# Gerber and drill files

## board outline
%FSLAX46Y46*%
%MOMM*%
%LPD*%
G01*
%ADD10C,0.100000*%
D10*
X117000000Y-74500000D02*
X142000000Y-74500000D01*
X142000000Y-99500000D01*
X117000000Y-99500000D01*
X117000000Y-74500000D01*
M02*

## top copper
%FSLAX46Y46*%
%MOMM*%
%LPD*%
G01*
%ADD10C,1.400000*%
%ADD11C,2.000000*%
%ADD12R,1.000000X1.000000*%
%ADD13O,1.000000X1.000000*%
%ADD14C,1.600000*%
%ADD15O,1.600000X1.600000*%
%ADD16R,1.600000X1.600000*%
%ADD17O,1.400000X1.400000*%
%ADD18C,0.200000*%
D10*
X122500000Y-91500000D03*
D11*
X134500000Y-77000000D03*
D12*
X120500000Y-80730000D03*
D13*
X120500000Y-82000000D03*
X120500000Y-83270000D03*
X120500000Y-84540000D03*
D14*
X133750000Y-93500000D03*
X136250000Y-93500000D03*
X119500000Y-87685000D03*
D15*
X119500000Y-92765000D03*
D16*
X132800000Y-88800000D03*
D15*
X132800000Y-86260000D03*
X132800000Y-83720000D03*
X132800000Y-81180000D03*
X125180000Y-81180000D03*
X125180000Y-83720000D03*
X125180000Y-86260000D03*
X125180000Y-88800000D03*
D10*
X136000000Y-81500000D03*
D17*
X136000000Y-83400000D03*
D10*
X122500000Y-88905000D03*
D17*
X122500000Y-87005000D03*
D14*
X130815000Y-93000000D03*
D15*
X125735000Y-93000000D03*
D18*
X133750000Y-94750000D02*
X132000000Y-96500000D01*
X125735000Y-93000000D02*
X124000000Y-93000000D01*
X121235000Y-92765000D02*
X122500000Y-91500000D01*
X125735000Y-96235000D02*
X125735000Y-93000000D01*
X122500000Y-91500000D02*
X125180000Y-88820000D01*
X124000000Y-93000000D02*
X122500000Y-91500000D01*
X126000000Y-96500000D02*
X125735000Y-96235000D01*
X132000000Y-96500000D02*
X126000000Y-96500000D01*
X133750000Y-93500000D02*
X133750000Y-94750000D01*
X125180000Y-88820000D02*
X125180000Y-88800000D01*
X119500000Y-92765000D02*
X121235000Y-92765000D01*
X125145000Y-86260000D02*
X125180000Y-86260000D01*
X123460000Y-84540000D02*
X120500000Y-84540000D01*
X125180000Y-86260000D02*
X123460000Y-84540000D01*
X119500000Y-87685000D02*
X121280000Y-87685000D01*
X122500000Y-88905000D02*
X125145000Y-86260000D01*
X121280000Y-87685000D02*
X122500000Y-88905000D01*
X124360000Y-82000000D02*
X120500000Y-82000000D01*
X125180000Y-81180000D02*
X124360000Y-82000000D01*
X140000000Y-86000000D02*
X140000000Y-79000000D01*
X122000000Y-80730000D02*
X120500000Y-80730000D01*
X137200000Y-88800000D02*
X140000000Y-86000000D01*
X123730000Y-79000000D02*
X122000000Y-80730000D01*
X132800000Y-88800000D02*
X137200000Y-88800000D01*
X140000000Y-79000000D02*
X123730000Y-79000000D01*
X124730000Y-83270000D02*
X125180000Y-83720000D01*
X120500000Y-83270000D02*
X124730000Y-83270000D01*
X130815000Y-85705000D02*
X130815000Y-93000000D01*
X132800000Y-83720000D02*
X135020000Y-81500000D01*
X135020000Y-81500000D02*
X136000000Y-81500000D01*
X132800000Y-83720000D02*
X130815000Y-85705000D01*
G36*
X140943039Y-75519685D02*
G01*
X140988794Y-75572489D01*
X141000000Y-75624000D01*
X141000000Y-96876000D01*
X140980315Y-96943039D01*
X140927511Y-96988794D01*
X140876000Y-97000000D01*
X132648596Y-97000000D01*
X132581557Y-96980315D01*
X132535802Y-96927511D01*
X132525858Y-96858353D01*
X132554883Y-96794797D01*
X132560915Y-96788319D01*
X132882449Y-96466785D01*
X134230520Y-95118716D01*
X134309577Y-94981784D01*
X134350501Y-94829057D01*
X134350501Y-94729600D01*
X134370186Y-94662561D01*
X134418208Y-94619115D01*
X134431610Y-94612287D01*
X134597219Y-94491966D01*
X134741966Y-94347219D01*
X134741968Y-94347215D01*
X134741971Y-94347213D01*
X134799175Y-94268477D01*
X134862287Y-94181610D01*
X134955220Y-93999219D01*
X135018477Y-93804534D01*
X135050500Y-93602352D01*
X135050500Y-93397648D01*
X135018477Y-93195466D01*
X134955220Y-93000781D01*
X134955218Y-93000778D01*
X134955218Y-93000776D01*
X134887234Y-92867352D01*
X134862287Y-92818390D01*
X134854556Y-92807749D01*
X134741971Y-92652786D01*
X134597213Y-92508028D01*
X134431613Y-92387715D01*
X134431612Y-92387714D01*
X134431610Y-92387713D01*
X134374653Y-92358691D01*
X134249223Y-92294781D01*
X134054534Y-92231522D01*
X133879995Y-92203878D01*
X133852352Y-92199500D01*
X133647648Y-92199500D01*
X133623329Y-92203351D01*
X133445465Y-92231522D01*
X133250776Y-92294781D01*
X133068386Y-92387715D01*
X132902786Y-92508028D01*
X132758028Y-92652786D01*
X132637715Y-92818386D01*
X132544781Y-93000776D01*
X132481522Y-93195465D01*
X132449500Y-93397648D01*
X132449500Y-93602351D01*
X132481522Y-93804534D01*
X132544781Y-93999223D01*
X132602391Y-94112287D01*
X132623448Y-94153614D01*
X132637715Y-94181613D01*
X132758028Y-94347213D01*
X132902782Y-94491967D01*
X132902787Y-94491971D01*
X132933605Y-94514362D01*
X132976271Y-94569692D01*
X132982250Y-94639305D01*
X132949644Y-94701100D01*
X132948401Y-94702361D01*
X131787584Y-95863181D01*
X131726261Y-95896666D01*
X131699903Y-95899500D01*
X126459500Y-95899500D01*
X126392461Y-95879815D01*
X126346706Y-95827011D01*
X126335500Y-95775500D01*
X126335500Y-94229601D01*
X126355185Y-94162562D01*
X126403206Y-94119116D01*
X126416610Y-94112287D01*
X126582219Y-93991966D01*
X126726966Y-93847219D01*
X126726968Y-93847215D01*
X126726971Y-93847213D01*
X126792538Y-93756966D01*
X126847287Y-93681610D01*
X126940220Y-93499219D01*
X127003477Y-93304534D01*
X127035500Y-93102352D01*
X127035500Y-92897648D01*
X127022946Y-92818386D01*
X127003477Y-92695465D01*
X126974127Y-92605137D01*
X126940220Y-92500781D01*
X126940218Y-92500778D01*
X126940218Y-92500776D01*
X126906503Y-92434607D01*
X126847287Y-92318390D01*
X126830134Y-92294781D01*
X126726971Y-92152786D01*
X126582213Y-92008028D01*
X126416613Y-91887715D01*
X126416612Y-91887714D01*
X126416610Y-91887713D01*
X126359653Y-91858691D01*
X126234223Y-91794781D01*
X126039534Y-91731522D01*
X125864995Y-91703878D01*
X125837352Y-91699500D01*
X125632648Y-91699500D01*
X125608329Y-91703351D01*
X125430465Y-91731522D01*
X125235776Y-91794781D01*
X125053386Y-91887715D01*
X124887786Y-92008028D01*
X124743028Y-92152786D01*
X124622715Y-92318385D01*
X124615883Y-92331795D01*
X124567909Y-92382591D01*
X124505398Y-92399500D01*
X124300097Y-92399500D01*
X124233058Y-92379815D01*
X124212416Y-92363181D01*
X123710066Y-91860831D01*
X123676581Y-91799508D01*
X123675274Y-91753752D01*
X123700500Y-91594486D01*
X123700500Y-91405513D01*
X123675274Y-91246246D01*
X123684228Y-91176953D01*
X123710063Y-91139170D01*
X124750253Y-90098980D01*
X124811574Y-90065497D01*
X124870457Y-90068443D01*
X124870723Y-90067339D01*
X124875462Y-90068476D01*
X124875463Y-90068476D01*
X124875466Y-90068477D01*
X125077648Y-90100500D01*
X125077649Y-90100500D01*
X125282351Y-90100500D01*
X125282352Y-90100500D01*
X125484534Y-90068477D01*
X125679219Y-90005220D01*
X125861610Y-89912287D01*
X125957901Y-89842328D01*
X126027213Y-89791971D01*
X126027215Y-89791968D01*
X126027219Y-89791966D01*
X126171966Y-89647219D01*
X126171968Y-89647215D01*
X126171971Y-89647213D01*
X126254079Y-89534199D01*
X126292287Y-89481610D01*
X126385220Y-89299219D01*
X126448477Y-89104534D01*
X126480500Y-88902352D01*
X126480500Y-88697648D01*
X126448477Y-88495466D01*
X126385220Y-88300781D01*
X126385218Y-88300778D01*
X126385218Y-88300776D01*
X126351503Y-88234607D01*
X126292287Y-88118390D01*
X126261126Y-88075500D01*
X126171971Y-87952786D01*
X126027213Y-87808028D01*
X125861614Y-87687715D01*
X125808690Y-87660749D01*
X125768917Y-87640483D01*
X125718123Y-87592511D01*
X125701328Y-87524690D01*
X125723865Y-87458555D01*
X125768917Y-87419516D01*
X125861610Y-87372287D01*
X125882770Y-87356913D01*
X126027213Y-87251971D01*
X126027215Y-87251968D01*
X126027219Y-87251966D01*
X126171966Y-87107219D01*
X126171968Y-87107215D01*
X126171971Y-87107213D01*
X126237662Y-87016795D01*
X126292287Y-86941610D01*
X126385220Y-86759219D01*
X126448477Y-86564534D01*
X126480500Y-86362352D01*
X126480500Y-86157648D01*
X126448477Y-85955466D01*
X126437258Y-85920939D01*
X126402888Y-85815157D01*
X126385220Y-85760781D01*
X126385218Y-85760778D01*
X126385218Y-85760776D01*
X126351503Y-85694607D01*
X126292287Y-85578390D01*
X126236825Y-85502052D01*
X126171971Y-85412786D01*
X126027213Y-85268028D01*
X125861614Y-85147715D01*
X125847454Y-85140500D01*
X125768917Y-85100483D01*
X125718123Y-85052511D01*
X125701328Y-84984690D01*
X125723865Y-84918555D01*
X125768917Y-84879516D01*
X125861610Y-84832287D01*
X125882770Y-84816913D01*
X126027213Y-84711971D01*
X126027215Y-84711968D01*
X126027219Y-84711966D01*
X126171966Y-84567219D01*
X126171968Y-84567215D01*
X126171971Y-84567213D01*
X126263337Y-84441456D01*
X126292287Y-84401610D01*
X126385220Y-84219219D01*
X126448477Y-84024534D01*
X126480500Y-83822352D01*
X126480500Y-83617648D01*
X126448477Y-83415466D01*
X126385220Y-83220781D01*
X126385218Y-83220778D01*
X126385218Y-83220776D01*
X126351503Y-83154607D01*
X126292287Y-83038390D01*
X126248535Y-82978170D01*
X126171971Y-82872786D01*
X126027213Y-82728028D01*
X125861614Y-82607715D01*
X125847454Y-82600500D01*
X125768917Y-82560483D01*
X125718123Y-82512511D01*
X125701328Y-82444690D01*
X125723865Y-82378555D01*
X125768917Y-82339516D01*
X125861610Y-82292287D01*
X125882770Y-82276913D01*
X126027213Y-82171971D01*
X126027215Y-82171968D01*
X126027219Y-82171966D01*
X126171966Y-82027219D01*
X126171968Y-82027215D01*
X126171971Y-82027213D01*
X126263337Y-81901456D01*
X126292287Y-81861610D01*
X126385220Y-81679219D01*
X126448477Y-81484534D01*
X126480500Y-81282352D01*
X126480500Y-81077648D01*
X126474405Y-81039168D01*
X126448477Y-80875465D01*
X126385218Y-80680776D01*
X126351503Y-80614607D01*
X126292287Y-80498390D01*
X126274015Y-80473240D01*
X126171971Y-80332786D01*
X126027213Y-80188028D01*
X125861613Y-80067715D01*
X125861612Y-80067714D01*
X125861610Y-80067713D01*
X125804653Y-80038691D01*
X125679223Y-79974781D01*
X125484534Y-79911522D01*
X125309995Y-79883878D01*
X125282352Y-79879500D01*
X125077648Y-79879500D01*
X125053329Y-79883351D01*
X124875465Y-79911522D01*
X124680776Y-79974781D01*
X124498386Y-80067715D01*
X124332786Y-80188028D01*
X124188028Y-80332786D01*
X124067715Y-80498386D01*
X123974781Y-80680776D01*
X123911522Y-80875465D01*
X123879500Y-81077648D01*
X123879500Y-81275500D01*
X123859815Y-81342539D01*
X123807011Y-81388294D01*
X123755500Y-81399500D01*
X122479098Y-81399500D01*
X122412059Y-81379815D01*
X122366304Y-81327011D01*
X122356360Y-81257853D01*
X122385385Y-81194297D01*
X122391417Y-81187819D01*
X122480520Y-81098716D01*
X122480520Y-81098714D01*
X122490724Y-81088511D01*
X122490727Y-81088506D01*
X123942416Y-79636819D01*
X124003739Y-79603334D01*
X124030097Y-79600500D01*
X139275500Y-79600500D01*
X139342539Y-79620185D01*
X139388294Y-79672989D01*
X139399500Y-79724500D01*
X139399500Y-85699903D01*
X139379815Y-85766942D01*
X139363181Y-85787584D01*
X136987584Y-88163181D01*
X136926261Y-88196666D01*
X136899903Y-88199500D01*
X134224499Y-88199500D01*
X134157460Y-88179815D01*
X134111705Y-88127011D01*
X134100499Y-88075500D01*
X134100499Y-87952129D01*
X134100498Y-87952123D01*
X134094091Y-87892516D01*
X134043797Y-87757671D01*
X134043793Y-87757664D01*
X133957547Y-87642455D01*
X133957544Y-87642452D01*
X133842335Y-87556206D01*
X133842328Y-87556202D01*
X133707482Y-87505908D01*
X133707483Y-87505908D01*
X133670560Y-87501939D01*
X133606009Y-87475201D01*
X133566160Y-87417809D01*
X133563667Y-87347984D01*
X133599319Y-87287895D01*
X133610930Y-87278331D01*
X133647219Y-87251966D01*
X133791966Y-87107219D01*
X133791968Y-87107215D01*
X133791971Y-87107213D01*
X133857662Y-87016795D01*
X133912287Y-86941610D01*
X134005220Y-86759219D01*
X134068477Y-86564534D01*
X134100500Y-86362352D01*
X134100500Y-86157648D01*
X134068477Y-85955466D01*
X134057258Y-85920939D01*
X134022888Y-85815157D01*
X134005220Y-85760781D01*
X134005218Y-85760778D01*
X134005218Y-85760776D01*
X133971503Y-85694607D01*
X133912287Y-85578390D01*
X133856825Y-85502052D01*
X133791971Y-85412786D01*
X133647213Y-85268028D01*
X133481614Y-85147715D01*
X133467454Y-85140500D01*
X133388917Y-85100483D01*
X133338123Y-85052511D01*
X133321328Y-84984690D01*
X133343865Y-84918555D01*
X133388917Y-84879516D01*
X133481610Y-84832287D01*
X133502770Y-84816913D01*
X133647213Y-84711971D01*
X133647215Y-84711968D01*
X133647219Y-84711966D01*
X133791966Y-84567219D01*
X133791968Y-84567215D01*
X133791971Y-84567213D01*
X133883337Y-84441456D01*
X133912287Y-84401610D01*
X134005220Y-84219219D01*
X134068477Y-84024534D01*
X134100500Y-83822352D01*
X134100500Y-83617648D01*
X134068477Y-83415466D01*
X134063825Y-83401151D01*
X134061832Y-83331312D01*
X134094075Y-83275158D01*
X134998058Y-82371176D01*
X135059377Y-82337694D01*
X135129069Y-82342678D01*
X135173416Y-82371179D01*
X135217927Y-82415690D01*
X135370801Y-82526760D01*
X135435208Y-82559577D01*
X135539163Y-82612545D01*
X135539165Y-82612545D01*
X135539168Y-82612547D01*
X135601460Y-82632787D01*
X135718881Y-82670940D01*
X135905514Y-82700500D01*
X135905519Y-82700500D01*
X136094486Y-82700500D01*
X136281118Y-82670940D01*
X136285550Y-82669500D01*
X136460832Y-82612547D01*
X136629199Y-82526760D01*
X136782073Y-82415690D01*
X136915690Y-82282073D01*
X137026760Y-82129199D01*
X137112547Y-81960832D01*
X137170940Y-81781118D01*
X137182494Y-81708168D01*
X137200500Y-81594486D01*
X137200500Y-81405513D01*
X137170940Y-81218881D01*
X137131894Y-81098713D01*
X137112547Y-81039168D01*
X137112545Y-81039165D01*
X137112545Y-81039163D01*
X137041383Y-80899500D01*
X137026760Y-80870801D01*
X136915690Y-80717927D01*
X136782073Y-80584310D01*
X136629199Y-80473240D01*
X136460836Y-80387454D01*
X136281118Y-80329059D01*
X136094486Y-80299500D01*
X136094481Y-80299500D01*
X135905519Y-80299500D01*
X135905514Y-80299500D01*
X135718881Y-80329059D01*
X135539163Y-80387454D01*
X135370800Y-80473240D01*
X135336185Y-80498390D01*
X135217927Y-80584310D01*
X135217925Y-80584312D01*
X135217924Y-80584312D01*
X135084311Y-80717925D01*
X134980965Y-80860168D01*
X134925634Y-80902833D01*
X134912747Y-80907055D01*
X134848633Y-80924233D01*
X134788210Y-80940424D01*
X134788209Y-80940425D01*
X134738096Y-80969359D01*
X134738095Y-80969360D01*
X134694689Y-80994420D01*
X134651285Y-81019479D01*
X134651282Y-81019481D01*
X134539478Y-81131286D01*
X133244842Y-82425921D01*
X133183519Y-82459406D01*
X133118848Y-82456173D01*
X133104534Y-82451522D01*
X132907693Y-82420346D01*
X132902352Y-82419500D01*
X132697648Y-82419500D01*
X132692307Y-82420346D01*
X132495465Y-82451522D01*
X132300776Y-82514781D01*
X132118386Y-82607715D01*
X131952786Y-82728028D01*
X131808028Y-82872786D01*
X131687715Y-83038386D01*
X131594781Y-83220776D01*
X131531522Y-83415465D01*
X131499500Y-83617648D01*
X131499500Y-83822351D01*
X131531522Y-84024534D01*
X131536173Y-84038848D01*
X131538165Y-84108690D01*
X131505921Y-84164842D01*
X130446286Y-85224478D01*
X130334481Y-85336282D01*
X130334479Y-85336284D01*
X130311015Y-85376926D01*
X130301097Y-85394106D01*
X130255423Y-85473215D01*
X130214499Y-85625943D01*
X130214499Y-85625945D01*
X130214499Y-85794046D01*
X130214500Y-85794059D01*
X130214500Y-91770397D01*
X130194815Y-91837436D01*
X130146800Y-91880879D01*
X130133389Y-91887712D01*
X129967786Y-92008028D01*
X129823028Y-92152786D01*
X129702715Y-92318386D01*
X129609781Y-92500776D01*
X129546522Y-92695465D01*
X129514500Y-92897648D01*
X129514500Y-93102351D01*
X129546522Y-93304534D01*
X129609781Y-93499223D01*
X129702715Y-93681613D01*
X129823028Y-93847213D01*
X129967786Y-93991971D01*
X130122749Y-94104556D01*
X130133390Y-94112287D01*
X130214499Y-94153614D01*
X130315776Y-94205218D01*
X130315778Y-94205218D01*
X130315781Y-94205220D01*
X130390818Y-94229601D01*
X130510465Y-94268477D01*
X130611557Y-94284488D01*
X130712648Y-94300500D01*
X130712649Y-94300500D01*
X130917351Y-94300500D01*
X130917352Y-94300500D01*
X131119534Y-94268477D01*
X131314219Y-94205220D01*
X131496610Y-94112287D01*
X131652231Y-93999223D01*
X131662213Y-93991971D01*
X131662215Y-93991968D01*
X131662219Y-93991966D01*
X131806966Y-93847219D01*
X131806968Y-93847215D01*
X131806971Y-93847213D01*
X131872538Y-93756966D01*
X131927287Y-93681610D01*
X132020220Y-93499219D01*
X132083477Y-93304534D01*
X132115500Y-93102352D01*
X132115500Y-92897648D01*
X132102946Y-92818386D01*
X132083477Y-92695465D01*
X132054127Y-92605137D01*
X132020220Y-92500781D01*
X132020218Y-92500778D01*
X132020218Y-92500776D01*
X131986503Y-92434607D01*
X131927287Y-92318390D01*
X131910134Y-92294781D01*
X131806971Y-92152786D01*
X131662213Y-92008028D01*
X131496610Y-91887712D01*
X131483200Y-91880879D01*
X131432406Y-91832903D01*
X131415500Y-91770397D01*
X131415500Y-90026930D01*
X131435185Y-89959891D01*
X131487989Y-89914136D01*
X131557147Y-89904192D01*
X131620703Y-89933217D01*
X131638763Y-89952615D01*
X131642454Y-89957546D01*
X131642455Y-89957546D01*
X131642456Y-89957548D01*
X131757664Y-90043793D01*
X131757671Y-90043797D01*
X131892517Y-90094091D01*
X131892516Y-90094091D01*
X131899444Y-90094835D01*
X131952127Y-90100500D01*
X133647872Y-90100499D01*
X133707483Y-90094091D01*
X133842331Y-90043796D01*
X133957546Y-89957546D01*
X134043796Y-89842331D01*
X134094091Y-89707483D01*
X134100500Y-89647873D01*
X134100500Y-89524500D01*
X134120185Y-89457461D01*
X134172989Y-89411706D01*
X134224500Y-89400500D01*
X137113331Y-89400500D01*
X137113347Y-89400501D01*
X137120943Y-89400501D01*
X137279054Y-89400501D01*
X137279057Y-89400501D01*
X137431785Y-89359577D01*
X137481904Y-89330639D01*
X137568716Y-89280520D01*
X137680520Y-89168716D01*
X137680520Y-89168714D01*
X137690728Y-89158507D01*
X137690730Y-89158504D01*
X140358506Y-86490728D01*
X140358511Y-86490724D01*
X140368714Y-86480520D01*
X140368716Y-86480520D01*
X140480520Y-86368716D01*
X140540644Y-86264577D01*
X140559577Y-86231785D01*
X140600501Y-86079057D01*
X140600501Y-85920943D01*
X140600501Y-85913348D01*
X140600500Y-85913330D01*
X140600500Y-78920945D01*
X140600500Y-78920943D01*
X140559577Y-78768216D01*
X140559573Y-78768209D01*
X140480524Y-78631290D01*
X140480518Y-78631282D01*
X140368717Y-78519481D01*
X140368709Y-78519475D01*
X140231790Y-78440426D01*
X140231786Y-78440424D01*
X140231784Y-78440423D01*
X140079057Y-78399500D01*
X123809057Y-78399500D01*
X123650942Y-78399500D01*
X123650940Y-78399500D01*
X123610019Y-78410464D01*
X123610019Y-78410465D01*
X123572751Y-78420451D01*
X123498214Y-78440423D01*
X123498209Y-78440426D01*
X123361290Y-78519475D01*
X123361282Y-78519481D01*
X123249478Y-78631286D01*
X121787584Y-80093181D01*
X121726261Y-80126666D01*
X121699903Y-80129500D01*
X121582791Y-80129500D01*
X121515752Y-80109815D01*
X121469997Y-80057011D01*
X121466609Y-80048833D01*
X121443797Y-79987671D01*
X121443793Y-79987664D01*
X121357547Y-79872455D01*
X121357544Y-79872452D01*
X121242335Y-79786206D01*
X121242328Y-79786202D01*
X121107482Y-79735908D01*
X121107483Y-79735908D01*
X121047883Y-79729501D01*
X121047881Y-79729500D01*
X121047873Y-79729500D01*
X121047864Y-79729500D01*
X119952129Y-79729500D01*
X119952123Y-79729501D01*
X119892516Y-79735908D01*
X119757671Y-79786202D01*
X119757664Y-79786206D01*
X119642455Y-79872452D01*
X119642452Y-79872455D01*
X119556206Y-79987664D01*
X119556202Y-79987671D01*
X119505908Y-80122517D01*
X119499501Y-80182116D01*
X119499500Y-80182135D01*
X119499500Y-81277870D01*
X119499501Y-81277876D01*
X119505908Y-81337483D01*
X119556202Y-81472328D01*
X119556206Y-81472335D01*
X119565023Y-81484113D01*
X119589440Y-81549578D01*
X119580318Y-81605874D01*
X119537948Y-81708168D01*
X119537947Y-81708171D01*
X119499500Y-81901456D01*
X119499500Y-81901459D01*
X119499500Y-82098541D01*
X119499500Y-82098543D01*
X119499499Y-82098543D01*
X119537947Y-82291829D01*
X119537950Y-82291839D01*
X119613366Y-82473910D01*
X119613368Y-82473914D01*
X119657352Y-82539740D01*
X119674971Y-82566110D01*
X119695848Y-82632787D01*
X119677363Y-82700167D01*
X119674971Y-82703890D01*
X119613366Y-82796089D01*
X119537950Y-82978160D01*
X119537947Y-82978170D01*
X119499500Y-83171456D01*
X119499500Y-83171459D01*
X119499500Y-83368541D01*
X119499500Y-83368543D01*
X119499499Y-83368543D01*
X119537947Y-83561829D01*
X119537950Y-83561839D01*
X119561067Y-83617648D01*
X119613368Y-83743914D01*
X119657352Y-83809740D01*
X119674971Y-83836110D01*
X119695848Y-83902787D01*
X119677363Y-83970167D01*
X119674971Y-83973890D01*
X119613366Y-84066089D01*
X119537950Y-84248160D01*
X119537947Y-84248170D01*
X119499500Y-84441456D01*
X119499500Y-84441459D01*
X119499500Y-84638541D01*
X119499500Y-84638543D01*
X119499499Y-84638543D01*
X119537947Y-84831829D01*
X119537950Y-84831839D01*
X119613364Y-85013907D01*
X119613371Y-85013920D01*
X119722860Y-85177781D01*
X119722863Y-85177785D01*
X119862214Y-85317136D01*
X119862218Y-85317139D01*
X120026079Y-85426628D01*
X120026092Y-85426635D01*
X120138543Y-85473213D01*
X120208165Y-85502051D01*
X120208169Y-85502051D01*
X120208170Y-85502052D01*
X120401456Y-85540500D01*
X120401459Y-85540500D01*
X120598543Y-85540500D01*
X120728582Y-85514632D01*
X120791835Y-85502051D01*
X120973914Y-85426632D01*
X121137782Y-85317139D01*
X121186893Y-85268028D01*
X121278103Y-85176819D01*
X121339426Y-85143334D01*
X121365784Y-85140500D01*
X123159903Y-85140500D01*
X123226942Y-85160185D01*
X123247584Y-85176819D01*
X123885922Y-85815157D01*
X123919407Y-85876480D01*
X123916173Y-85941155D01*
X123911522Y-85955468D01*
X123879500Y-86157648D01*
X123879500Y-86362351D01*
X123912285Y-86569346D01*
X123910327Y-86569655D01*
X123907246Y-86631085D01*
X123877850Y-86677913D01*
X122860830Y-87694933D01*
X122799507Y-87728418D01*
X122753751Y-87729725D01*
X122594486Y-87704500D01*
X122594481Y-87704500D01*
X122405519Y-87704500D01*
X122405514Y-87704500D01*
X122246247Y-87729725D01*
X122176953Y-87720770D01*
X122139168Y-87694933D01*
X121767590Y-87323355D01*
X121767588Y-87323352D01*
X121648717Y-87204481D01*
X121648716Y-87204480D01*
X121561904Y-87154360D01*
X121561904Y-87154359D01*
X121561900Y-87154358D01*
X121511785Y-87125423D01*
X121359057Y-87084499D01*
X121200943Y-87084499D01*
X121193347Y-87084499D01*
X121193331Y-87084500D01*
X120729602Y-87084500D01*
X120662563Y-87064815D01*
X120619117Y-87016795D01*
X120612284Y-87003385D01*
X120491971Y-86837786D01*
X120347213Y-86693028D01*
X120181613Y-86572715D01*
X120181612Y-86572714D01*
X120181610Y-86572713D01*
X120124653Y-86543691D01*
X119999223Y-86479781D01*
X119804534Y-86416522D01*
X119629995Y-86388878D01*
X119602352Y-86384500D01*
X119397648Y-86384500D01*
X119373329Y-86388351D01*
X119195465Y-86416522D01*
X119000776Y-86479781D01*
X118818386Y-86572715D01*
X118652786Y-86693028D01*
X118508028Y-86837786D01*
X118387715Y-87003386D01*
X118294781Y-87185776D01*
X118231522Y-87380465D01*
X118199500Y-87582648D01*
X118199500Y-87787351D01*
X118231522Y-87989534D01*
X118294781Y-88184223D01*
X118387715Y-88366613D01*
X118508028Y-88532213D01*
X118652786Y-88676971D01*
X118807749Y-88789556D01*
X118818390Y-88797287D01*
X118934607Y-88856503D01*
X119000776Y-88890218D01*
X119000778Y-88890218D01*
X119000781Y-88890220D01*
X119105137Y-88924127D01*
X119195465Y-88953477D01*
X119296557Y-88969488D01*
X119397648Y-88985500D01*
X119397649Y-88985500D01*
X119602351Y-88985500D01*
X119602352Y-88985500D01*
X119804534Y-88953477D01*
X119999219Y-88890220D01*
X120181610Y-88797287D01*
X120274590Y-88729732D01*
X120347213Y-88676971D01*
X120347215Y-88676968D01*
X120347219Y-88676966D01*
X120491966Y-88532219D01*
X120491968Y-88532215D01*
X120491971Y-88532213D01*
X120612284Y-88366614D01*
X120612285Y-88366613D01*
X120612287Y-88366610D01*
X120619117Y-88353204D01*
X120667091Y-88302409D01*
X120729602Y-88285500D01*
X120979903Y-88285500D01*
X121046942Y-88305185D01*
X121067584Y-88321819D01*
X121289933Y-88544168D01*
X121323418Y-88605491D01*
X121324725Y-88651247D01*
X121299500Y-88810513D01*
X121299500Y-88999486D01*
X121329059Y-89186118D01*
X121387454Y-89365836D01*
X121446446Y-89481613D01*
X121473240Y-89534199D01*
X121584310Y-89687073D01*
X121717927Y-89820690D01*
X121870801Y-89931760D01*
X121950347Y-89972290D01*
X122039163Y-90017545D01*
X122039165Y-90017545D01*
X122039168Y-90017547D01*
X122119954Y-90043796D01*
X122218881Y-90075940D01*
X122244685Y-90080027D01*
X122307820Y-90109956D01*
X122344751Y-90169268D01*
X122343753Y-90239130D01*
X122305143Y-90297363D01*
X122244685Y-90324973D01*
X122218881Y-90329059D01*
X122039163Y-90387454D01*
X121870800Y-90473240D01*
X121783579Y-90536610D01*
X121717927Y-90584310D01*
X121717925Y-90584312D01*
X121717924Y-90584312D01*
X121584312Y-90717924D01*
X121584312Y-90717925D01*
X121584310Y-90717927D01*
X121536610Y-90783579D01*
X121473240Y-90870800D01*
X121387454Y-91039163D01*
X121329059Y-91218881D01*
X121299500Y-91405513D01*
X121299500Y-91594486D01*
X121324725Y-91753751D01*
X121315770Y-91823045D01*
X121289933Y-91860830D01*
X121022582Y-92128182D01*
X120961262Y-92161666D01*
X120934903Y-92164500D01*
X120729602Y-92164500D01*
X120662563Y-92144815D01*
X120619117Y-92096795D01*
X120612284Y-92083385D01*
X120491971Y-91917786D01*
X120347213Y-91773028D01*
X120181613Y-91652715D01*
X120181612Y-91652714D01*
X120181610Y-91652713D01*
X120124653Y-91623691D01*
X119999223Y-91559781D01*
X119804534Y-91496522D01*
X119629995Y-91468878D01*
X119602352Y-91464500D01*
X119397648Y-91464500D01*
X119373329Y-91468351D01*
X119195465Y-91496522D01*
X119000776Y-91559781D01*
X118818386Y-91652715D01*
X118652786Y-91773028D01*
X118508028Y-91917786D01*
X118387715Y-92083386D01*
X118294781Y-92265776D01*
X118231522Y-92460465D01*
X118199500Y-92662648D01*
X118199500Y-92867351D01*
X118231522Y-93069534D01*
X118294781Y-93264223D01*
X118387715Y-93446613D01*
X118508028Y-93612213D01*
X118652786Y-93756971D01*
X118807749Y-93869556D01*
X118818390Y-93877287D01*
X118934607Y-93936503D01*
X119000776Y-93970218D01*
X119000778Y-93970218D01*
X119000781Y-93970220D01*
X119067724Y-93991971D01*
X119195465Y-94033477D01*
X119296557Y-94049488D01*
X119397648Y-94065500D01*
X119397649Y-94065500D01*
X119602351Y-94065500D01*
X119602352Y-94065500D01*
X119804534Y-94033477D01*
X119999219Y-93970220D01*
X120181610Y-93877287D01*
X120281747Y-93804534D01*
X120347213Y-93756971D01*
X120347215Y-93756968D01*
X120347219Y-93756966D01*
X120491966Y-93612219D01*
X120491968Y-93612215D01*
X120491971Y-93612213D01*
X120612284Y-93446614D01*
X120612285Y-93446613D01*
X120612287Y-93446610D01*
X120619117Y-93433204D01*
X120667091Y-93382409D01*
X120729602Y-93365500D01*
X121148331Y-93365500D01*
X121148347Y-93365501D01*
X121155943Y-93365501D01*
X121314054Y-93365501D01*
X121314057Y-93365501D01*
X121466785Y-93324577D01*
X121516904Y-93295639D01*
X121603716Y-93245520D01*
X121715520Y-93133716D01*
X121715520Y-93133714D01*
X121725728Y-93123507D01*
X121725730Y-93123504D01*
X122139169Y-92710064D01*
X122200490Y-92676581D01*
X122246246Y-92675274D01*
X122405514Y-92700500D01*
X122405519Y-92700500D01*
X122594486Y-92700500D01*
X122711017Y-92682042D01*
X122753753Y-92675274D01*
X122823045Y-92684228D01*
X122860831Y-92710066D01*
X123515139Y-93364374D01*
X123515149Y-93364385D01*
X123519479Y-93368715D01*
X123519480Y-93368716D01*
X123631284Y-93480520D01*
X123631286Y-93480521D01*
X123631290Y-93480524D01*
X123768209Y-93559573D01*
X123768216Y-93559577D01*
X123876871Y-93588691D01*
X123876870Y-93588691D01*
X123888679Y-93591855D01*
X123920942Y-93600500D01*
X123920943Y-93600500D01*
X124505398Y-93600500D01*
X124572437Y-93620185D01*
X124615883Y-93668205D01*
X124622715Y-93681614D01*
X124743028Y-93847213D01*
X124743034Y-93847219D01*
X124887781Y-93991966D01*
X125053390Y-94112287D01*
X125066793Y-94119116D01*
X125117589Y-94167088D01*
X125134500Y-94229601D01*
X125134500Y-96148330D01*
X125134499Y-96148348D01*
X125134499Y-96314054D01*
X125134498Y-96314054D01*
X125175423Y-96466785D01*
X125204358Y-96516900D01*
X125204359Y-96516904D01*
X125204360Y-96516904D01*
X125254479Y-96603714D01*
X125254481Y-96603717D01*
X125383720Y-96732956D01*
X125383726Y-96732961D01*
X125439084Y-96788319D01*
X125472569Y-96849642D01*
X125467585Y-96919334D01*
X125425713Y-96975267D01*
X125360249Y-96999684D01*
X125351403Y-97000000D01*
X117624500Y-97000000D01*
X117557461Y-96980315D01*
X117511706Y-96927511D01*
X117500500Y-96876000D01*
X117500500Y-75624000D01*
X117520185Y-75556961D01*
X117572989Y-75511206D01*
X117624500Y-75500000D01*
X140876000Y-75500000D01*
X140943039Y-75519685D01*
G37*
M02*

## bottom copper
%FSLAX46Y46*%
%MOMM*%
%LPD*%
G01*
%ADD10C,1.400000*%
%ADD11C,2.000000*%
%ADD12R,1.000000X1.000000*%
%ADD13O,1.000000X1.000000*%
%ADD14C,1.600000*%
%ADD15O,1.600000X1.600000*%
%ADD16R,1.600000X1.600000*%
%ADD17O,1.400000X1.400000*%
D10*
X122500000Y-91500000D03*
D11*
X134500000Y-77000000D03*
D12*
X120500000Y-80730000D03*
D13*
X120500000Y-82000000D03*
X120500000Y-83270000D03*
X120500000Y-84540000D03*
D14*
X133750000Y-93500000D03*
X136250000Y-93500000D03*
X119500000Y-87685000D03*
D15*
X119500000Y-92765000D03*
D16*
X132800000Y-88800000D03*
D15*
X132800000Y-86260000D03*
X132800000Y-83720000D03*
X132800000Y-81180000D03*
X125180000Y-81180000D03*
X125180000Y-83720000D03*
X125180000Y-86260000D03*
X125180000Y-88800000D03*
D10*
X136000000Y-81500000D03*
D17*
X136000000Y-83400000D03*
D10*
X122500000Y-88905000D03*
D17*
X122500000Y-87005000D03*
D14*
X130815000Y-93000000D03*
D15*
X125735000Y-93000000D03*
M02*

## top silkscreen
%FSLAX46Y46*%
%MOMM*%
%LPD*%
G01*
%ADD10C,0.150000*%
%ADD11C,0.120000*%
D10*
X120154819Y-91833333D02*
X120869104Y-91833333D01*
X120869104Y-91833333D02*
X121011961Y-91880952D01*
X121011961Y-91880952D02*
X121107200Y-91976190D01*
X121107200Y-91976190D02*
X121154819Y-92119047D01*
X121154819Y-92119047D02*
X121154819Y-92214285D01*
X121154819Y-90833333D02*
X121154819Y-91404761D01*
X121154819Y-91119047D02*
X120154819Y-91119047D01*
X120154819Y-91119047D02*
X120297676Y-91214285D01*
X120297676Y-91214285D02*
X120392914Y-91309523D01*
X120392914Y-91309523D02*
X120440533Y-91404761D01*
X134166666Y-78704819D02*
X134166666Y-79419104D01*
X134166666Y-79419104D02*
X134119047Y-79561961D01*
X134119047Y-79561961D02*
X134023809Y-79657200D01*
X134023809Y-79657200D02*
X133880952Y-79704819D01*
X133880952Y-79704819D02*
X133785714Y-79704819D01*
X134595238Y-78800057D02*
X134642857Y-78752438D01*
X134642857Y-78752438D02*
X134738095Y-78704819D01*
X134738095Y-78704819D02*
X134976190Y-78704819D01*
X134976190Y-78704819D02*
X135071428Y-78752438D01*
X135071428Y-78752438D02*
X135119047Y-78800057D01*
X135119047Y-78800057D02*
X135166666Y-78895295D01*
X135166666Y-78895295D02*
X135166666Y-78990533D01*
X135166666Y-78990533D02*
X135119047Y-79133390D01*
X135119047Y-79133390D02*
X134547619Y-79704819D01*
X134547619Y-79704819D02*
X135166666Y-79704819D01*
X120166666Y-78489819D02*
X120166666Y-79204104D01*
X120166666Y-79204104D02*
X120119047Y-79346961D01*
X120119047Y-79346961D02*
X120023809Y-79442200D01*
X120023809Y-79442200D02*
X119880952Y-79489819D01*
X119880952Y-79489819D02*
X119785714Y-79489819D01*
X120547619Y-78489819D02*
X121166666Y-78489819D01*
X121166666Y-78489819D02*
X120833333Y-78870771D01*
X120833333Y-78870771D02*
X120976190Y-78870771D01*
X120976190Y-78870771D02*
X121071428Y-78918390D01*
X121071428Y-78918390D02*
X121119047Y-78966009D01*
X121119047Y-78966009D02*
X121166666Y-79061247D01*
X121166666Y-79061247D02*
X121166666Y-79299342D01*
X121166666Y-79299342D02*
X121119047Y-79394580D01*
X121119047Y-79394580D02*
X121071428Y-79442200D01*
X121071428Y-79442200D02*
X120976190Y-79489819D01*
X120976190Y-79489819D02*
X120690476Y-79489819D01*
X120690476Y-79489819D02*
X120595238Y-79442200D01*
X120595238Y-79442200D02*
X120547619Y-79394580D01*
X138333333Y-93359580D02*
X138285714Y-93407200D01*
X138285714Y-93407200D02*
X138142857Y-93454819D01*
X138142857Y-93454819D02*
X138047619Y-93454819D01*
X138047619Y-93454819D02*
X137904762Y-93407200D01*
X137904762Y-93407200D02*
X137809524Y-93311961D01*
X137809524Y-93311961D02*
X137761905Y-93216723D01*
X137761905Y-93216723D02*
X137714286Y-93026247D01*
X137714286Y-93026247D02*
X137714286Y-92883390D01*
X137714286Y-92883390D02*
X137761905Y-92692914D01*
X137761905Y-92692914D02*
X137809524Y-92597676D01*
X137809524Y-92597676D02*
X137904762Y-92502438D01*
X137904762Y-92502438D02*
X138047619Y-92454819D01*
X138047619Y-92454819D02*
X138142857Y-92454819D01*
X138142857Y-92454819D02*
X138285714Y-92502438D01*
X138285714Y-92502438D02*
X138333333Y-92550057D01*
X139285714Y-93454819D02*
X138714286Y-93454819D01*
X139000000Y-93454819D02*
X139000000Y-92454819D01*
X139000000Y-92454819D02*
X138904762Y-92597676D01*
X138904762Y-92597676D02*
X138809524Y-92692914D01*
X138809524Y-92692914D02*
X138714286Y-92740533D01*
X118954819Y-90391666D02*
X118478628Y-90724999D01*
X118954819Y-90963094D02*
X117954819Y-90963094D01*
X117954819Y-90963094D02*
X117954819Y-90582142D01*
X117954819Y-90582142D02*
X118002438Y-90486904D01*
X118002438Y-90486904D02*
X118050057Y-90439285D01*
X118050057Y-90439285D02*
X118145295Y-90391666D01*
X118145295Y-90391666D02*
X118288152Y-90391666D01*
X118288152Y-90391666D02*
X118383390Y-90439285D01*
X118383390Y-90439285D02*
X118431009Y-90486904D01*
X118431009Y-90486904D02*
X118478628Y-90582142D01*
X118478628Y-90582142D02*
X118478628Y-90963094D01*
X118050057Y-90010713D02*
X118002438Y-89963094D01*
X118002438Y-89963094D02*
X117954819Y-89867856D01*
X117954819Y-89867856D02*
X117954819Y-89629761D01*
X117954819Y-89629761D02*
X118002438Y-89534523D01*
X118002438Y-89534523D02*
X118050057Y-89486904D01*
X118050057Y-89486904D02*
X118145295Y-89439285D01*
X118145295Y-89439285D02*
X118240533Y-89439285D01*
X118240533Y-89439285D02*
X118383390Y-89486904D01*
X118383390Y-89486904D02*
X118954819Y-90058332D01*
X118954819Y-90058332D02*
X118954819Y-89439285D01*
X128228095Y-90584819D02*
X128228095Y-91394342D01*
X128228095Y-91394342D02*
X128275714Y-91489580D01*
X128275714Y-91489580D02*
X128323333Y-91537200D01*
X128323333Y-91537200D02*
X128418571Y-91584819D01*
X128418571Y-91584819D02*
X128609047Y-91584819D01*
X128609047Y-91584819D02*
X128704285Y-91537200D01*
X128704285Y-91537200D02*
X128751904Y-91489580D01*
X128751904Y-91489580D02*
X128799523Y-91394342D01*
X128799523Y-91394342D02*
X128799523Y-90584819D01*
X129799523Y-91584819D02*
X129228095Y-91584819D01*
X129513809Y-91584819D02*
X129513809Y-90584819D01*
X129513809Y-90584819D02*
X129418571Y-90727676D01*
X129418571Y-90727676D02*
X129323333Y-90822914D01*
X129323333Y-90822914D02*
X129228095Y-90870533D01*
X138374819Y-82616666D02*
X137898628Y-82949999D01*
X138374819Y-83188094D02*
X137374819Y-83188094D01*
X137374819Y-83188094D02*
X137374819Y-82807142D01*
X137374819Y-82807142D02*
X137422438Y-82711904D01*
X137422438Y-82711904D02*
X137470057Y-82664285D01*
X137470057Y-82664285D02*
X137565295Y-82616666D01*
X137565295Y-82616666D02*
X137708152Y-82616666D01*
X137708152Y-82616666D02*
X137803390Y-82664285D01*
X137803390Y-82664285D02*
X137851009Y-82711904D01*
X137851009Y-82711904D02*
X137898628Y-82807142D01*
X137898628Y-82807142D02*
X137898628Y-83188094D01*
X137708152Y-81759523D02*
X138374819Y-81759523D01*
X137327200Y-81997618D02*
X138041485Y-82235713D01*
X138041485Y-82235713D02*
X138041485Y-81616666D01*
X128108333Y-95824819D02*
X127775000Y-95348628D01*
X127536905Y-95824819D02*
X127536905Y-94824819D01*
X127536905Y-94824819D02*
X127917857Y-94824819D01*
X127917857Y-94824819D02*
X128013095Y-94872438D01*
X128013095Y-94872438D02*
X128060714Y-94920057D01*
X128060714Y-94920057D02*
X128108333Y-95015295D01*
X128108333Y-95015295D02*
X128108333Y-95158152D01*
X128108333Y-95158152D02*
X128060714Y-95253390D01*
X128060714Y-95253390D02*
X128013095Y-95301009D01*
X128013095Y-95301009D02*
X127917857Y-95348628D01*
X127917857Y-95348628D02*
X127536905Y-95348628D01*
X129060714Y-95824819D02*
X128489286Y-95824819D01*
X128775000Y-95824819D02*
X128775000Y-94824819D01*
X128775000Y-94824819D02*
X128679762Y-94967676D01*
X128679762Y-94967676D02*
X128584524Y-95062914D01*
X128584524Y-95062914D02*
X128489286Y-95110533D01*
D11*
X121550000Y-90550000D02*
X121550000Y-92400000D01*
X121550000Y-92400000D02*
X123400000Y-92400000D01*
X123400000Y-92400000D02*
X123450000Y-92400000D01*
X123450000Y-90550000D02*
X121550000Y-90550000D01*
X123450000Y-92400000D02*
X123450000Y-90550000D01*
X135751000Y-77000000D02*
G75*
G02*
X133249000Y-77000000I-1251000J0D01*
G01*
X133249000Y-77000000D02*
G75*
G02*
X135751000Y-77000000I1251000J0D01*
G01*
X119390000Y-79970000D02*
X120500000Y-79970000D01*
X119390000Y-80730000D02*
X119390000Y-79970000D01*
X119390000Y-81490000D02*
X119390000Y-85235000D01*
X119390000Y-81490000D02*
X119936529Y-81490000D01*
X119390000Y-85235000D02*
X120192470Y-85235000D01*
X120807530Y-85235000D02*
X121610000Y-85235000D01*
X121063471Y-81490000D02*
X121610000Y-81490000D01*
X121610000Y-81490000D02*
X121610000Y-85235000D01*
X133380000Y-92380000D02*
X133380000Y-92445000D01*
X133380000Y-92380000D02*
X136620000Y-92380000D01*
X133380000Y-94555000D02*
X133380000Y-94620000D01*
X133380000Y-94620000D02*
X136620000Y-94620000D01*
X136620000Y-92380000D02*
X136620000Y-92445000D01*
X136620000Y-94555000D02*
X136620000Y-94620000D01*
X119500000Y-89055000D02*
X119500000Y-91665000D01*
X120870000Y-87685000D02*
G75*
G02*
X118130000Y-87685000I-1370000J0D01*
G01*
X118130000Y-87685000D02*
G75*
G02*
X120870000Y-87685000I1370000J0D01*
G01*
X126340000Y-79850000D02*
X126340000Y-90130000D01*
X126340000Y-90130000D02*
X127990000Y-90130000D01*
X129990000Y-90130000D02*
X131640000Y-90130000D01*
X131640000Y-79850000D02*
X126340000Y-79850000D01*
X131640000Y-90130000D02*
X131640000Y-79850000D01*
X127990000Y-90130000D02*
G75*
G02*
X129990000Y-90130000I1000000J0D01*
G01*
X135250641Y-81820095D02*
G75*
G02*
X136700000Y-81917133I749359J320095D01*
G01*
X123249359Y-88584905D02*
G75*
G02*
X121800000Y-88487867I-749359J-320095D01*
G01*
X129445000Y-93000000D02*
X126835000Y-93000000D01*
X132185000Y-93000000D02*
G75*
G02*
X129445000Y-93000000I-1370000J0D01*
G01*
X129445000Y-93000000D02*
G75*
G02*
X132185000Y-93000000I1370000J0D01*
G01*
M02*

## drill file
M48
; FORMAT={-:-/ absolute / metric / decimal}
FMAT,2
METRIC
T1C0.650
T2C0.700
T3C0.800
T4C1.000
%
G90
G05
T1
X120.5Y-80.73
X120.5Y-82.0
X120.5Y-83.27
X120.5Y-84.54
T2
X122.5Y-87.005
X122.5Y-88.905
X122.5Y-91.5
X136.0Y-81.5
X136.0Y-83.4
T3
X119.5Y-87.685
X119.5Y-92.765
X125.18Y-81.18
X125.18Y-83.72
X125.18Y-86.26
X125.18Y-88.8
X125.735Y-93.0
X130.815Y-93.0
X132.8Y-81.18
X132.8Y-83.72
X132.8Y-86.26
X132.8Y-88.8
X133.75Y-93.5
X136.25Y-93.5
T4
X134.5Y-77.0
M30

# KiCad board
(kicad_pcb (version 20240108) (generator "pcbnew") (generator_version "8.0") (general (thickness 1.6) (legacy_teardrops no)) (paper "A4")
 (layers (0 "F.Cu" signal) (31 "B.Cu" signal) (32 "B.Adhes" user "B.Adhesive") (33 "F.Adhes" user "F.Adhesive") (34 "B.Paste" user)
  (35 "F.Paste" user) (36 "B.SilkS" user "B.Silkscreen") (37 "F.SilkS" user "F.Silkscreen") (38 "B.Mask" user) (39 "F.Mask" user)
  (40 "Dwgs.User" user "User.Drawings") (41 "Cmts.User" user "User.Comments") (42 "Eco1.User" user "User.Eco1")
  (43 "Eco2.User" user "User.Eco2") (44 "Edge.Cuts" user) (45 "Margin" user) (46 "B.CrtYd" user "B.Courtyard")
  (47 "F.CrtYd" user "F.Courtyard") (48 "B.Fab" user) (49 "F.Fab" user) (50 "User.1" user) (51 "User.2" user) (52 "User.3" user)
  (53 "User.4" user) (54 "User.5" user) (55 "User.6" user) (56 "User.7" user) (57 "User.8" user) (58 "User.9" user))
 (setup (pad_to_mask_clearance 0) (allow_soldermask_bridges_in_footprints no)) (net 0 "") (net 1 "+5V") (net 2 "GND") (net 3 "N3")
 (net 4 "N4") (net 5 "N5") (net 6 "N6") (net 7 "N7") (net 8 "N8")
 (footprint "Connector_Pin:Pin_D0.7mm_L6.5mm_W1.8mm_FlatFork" (layer "F.Cu") (at 122.5 91.5 -90)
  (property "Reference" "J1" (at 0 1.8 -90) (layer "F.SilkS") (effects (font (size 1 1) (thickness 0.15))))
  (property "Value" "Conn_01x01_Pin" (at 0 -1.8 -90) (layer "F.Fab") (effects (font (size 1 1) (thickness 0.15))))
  (fp_line (start -0.95 0.95) (end 0.9 0.95) (stroke (width 0.12) (type solid)) (layer "F.SilkS"))
  (fp_line (start 0.9 0.95) (end 0.9 -0.9) (stroke (width 0.12) (type solid)) (layer "F.SilkS"))
  (fp_line (start 0.9 -0.9) (end 0.9 -0.95) (stroke (width 0.12) (type solid)) (layer "F.SilkS"))
  (fp_line (start -0.95 -0.95) (end -0.95 0.95) (stroke (width 0.12) (type solid)) (layer "F.SilkS"))
  (fp_line (start 0.9 -0.95) (end -0.95 -0.95) (stroke (width 0.12) (type solid)) (layer "F.SilkS"))
  (pad "1" thru_hole circle (at 0 0 270) (size 1.4 1.4) (drill 0.7) (layers "*.Cu" "*.Mask") (remove_unused_layers no) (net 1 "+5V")))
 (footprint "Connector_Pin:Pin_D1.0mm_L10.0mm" (layer "F.Cu") (at 134.5 77)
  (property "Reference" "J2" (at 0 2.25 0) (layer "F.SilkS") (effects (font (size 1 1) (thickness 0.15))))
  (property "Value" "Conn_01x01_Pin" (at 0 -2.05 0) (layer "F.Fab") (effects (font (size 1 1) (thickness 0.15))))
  (fp_circle (center 0 0) (end 1.25 0.05) (stroke (width 0.12) (type solid)) (fill none) (layer "F.SilkS"))
  (pad "1" thru_hole circle (at 0 0) (size 2 2) (drill 1) (layers "*.Cu" "*.Mask") (remove_unused_layers no) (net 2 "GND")))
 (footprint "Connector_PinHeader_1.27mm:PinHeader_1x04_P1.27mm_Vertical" (layer "F.Cu") (at 120.5 80.73)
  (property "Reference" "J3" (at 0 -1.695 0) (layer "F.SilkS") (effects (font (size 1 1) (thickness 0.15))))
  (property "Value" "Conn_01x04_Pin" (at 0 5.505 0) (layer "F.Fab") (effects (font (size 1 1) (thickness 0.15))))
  (fp_line (start -1.11 -0.76) (end 0 -0.76) (stroke (width 0.12) (type solid)) (layer "F.SilkS"))
  (fp_line (start -1.11 0) (end -1.11 -0.76) (stroke (width 0.12) (type solid)) (layer "F.SilkS"))
  (fp_line (start -1.11 0.76) (end -1.11 4.505) (stroke (width 0.12) (type solid)) (layer "F.SilkS"))
  (fp_line (start -1.11 0.76) (end -0.563471 0.76) (stroke (width 0.12) (type solid)) (layer "F.SilkS"))
  (fp_line (start -1.11 4.505) (end -0.30753 4.505) (stroke (width 0.12) (type solid)) (layer "F.SilkS"))
  (fp_line (start 0.30753 4.505) (end 1.11 4.505) (stroke (width 0.12) (type solid)) (layer "F.SilkS"))
  (fp_line (start 0.563471 0.76) (end 1.11 0.76) (stroke (width 0.12) (type solid)) (layer "F.SilkS"))
  (fp_line (start 1.11 0.76) (end 1.11 4.505) (stroke (width 0.12) (type solid)) (layer "F.SilkS"))
  (pad "1" thru_hole rect (at 0 0) (size 1 1) (drill 0.65) (layers "*.Cu" "*.Mask") (remove_unused_layers no) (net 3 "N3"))
  (pad "2" thru_hole oval (at 0 1.27) (size 1 1) (drill 0.65) (layers "*.Cu" "*.Mask") (remove_unused_layers no) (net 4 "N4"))
  (pad "3" thru_hole oval (at 0 2.54) (size 1 1) (drill 0.65) (layers "*.Cu" "*.Mask") (remove_unused_layers no) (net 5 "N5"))
  (pad "4" thru_hole oval (at 0 3.81) (size 1 1) (drill 0.65) (layers "*.Cu" "*.Mask") (remove_unused_layers no) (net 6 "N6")))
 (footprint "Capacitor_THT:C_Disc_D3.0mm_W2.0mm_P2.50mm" (layer "F.Cu") (at 133.75 93.5)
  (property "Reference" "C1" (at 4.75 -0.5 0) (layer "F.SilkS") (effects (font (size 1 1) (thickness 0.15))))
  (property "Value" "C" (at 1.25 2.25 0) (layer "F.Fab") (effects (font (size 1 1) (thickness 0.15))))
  (fp_line (start -0.37 -1.12) (end -0.37 -1.055) (stroke (width 0.12) (type solid)) (layer "F.SilkS"))
  (fp_line (start -0.37 -1.12) (end 2.87 -1.12) (stroke (width 0.12) (type solid)) (layer "F.SilkS"))
  (fp_line (start -0.37 1.055) (end -0.37 1.12) (stroke (width 0.12) (type solid)) (layer "F.SilkS"))
  (fp_line (start -0.37 1.12) (end 2.87 1.12) (stroke (width 0.12) (type solid)) (layer "F.SilkS"))
  (fp_line (start 2.87 -1.12) (end 2.87 -1.055) (stroke (width 0.12) (type solid)) (layer "F.SilkS"))
  (fp_line (start 2.87 1.055) (end 2.87 1.12) (stroke (width 0.12) (type solid)) (layer "F.SilkS"))
  (pad "1" thru_hole circle (at 0 0) (size 1.6 1.6) (drill 0.8) (layers "*.Cu" "*.Mask") (remove_unused_layers no) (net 1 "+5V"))
  (pad "2" thru_hole circle (at 2.5 0) (size 1.6 1.6) (drill 0.8) (layers "*.Cu" "*.Mask") (remove_unused_layers no) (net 2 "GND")))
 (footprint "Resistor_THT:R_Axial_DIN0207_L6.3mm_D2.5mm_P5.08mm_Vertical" (layer "F.Cu") (at 119.5 87.685 -90)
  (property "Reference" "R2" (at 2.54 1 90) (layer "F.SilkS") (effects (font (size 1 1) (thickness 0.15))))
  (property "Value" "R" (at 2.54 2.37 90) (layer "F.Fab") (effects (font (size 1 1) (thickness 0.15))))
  (fp_line (start 1.37 0) (end 3.98 0) (stroke (width 0.12) (type solid)) (layer "F.SilkS"))
  (fp_circle (center 0 0) (end 1.37 0) (stroke (width 0.12) (type solid)) (fill none) (layer "F.SilkS"))
  (pad "1" thru_hole circle (at 0 0 270) (size 1.6 1.6) (drill 0.8) (layers "*.Cu" "*.Mask") (remove_unused_layers no) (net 6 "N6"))
  (pad "2" thru_hole oval (at 5.08 0 270) (size 1.6 1.6) (drill 0.8) (layers "*.Cu" "*.Mask") (remove_unused_layers no) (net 1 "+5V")))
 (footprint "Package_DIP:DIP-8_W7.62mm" (layer "F.Cu") (at 132.8 88.8 180)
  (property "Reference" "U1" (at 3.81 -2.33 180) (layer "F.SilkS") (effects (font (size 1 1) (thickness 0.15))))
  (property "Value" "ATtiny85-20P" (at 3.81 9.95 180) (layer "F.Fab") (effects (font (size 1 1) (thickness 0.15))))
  (fp_line (start 6.46 8.95) (end 6.46 -1.33) (stroke (width 0.12) (type solid)) (layer "F.SilkS"))
  (fp_line (start 6.46 -1.33) (end 4.81 -1.33) (stroke (width 0.12) (type solid)) (layer "F.SilkS"))
  (fp_line (start 2.81 -1.33) (end 1.16 -1.33) (stroke (width 0.12) (type solid)) (layer "F.SilkS"))
  (fp_line (start 1.16 8.95) (end 6.46 8.95) (stroke (width 0.12) (type solid)) (layer "F.SilkS"))
  (fp_line (start 1.16 -1.33) (end 1.16 8.95) (stroke (width 0.12) (type solid)) (layer "F.SilkS"))
  (fp_arc (start 4.81 -1.33) (mid 3.81 -0.33) (end 2.81 -1.33) (stroke (width 0.12) (type solid)) (layer "F.SilkS"))
  (pad "1" thru_hole rect (at 0 0 180) (size 1.6 1.6) (drill 0.8) (layers "*.Cu" "*.Mask") (remove_unused_layers no) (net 3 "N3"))
  (pad "2" thru_hole oval (at 0 2.54 180) (size 1.6 1.6) (drill 0.8) (layers "*.Cu" "*.Mask") (remove_unused_layers no) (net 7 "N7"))
  (pad "3" thru_hole oval (at 0 5.08 180) (size 1.6 1.6) (drill 0.8) (layers "*.Cu" "*.Mask") (remove_unused_layers no) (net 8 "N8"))
  (pad "4" thru_hole oval (at 0 7.62 180) (size 1.6 1.6) (drill 0.8) (layers "*.Cu" "*.Mask") (remove_unused_layers no) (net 2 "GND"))
  (pad "5" thru_hole oval (at 7.62 7.62 180) (size 1.6 1.6) (drill 0.8) (layers "*.Cu" "*.Mask") (remove_unused_layers no) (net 4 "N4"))
  (pad "6" thru_hole oval (at 7.62 5.08 180) (size 1.6 1.6) (drill 0.8) (layers "*.Cu" "*.Mask") (remove_unused_layers no) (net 5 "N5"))
  (pad "7" thru_hole oval (at 7.62 2.54 180) (size 1.6 1.6) (drill 0.8) (layers "*.Cu" "*.Mask") (remove_unused_layers no) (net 6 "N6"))
  (pad "8" thru_hole oval (at 7.62 0 180) (size 1.6 1.6) (drill 0.8) (layers "*.Cu" "*.Mask") (remove_unused_layers no) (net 1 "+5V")))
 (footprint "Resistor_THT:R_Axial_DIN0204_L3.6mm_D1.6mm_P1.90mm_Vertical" (layer "F.Cu") (at 136 81.5 -90)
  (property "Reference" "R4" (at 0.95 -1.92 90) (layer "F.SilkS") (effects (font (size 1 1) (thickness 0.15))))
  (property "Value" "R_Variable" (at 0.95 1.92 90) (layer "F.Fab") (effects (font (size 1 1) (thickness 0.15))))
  (fp_arc (start 0.320095 0.749359) (mid -0.813042 -0.054435) (end 0.417133 -0.7) (stroke (width 0.12) (type solid)) (layer "F.SilkS"))
  (pad "1" thru_hole circle (at 0 0 270) (size 1.4 1.4) (drill 0.7) (layers "*.Cu" "*.Mask") (remove_unused_layers no) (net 8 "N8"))
  (pad "2" thru_hole oval (at 1.9 0 270) (size 1.4 1.4) (drill 0.7) (layers "*.Cu" "*.Mask") (remove_unused_layers no) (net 2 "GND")))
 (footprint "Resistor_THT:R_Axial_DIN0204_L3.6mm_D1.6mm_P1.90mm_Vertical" (layer "F.Cu") (at 122.5 88.905 90)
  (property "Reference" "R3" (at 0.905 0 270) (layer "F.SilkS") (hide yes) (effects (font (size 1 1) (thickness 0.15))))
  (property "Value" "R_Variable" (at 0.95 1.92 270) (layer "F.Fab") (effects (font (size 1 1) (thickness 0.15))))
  (fp_arc (start 0.320095 0.749359) (mid -0.813042 -0.054435) (end 0.417133 -0.7) (stroke (width 0.12) (type solid)) (layer "F.SilkS"))
  (pad "1" thru_hole circle (at 0 0 90) (size 1.4 1.4) (drill 0.7) (layers "*.Cu" "*.Mask") (remove_unused_layers no) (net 6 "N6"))
  (pad "2" thru_hole oval (at 1.9 0 90) (size 1.4 1.4) (drill 0.7) (layers "*.Cu" "*.Mask") (remove_unused_layers no) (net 2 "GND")))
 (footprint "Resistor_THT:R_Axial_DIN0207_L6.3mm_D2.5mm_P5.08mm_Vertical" (layer "F.Cu") (at 130.815 93 180)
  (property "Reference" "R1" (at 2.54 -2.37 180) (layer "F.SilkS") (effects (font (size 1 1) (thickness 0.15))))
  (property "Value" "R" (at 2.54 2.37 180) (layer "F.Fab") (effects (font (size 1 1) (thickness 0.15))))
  (fp_line (start 1.37 0) (end 3.98 0) (stroke (width 0.12) (type solid)) (layer "F.SilkS"))
  (fp_circle (center 0 0) (end 1.37 0) (stroke (width 0.12) (type solid)) (fill none) (layer "F.SilkS"))
  (pad "1" thru_hole circle (at 0 0 180) (size 1.6 1.6) (drill 0.8) (layers "*.Cu" "*.Mask") (remove_unused_layers no) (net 8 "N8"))
  (pad "2" thru_hole oval (at 5.08 0 180) (size 1.6 1.6) (drill 0.8) (layers "*.Cu" "*.Mask") (remove_unused_layers no) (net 1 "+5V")))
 (gr_rect (start 117 74.5) (end 142 99.5) (stroke (width 0.1) (type default)) (fill none) (layer "Edge.Cuts"))
 (segment (start 133.75 94.75) (end 132 96.5) (width 0.2) (layer "F.Cu") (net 1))
 (segment (start 125.735 93) (end 124 93) (width 0.2) (layer "F.Cu") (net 1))
 (segment (start 121.235 92.765) (end 122.5 91.5) (width 0.2) (layer "F.Cu") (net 1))
 (segment (start 125.735 96.235) (end 125.735 93) (width 0.2) (layer "F.Cu") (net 1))
 (segment (start 122.5 91.5) (end 125.18 88.82) (width 0.2) (layer "F.Cu") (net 1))
 (segment (start 124 93) (end 122.5 91.5) (width 0.2) (layer "F.Cu") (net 1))
 (segment (start 126 96.5) (end 125.735 96.235) (width 0.2) (layer "F.Cu") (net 1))
 (segment (start 132 96.5) (end 126 96.5) (width 0.2) (layer "F.Cu") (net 1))
 (segment (start 133.75 93.5) (end 133.75 94.75) (width 0.2) (layer "F.Cu") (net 1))
 (segment (start 125.18 88.82) (end 125.18 88.8) (width 0.2) (layer "F.Cu") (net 1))
 (segment (start 119.5 92.765) (end 121.235 92.765) (width 0.2) (layer "F.Cu") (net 1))
 (segment (start 125.145 86.26) (end 125.18 86.26) (width 0.2) (layer "F.Cu") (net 6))
 (segment (start 123.46 84.54) (end 120.5 84.54) (width 0.2) (layer "F.Cu") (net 6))
 (segment (start 125.18 86.26) (end 123.46 84.54) (width 0.2) (layer "F.Cu") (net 6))
 (segment (start 119.5 87.685) (end 121.28 87.685) (width 0.2) (layer "F.Cu") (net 6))
 (segment (start 122.5 88.905) (end 125.145 86.26) (width 0.2) (layer "F.Cu") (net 6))
 (segment (start 121.28 87.685) (end 122.5 88.905) (width 0.2) (layer "F.Cu") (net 6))
 (segment (start 124.36 82) (end 120.5 82) (width 0.2) (layer "F.Cu") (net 4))
 (segment (start 125.18 81.18) (end 124.36 82) (width 0.2) (layer "F.Cu") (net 4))
 (segment (start 140 86) (end 140 79) (width 0.2) (layer "F.Cu") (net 3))
 (segment (start 122 80.73) (end 120.5 80.73) (width 0.2) (layer "F.Cu") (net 3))
 (segment (start 137.2 88.8) (end 140 86) (width 0.2) (layer "F.Cu") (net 3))
 (segment (start 123.73 79) (end 122 80.73) (width 0.2) (layer "F.Cu") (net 3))
 (segment (start 132.8 88.8) (end 137.2 88.8) (width 0.2) (layer "F.Cu") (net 3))
 (segment (start 140 79) (end 123.73 79) (width 0.2) (layer "F.Cu") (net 3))
 (segment (start 124.73 83.27) (end 125.18 83.72) (width 0.2) (layer "F.Cu") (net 5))
 (segment (start 120.5 83.27) (end 124.73 83.27) (width 0.2) (layer "F.Cu") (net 5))
 (segment (start 130.815 85.705) (end 130.815 93) (width 0.2) (layer "F.Cu") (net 8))
 (segment (start 132.8 83.72) (end 135.02 81.5) (width 0.2) (layer "F.Cu") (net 8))
 (segment (start 135.02 81.5) (end 136 81.5) (width 0.2) (layer "F.Cu") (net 8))
 (segment (start 132.8 83.72) (end 130.815 85.705) (width 0.2) (layer "F.Cu") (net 8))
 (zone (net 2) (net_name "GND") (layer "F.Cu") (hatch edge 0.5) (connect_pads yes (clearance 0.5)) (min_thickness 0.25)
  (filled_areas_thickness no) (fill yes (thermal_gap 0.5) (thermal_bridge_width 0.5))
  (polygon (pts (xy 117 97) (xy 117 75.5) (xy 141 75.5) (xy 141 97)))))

